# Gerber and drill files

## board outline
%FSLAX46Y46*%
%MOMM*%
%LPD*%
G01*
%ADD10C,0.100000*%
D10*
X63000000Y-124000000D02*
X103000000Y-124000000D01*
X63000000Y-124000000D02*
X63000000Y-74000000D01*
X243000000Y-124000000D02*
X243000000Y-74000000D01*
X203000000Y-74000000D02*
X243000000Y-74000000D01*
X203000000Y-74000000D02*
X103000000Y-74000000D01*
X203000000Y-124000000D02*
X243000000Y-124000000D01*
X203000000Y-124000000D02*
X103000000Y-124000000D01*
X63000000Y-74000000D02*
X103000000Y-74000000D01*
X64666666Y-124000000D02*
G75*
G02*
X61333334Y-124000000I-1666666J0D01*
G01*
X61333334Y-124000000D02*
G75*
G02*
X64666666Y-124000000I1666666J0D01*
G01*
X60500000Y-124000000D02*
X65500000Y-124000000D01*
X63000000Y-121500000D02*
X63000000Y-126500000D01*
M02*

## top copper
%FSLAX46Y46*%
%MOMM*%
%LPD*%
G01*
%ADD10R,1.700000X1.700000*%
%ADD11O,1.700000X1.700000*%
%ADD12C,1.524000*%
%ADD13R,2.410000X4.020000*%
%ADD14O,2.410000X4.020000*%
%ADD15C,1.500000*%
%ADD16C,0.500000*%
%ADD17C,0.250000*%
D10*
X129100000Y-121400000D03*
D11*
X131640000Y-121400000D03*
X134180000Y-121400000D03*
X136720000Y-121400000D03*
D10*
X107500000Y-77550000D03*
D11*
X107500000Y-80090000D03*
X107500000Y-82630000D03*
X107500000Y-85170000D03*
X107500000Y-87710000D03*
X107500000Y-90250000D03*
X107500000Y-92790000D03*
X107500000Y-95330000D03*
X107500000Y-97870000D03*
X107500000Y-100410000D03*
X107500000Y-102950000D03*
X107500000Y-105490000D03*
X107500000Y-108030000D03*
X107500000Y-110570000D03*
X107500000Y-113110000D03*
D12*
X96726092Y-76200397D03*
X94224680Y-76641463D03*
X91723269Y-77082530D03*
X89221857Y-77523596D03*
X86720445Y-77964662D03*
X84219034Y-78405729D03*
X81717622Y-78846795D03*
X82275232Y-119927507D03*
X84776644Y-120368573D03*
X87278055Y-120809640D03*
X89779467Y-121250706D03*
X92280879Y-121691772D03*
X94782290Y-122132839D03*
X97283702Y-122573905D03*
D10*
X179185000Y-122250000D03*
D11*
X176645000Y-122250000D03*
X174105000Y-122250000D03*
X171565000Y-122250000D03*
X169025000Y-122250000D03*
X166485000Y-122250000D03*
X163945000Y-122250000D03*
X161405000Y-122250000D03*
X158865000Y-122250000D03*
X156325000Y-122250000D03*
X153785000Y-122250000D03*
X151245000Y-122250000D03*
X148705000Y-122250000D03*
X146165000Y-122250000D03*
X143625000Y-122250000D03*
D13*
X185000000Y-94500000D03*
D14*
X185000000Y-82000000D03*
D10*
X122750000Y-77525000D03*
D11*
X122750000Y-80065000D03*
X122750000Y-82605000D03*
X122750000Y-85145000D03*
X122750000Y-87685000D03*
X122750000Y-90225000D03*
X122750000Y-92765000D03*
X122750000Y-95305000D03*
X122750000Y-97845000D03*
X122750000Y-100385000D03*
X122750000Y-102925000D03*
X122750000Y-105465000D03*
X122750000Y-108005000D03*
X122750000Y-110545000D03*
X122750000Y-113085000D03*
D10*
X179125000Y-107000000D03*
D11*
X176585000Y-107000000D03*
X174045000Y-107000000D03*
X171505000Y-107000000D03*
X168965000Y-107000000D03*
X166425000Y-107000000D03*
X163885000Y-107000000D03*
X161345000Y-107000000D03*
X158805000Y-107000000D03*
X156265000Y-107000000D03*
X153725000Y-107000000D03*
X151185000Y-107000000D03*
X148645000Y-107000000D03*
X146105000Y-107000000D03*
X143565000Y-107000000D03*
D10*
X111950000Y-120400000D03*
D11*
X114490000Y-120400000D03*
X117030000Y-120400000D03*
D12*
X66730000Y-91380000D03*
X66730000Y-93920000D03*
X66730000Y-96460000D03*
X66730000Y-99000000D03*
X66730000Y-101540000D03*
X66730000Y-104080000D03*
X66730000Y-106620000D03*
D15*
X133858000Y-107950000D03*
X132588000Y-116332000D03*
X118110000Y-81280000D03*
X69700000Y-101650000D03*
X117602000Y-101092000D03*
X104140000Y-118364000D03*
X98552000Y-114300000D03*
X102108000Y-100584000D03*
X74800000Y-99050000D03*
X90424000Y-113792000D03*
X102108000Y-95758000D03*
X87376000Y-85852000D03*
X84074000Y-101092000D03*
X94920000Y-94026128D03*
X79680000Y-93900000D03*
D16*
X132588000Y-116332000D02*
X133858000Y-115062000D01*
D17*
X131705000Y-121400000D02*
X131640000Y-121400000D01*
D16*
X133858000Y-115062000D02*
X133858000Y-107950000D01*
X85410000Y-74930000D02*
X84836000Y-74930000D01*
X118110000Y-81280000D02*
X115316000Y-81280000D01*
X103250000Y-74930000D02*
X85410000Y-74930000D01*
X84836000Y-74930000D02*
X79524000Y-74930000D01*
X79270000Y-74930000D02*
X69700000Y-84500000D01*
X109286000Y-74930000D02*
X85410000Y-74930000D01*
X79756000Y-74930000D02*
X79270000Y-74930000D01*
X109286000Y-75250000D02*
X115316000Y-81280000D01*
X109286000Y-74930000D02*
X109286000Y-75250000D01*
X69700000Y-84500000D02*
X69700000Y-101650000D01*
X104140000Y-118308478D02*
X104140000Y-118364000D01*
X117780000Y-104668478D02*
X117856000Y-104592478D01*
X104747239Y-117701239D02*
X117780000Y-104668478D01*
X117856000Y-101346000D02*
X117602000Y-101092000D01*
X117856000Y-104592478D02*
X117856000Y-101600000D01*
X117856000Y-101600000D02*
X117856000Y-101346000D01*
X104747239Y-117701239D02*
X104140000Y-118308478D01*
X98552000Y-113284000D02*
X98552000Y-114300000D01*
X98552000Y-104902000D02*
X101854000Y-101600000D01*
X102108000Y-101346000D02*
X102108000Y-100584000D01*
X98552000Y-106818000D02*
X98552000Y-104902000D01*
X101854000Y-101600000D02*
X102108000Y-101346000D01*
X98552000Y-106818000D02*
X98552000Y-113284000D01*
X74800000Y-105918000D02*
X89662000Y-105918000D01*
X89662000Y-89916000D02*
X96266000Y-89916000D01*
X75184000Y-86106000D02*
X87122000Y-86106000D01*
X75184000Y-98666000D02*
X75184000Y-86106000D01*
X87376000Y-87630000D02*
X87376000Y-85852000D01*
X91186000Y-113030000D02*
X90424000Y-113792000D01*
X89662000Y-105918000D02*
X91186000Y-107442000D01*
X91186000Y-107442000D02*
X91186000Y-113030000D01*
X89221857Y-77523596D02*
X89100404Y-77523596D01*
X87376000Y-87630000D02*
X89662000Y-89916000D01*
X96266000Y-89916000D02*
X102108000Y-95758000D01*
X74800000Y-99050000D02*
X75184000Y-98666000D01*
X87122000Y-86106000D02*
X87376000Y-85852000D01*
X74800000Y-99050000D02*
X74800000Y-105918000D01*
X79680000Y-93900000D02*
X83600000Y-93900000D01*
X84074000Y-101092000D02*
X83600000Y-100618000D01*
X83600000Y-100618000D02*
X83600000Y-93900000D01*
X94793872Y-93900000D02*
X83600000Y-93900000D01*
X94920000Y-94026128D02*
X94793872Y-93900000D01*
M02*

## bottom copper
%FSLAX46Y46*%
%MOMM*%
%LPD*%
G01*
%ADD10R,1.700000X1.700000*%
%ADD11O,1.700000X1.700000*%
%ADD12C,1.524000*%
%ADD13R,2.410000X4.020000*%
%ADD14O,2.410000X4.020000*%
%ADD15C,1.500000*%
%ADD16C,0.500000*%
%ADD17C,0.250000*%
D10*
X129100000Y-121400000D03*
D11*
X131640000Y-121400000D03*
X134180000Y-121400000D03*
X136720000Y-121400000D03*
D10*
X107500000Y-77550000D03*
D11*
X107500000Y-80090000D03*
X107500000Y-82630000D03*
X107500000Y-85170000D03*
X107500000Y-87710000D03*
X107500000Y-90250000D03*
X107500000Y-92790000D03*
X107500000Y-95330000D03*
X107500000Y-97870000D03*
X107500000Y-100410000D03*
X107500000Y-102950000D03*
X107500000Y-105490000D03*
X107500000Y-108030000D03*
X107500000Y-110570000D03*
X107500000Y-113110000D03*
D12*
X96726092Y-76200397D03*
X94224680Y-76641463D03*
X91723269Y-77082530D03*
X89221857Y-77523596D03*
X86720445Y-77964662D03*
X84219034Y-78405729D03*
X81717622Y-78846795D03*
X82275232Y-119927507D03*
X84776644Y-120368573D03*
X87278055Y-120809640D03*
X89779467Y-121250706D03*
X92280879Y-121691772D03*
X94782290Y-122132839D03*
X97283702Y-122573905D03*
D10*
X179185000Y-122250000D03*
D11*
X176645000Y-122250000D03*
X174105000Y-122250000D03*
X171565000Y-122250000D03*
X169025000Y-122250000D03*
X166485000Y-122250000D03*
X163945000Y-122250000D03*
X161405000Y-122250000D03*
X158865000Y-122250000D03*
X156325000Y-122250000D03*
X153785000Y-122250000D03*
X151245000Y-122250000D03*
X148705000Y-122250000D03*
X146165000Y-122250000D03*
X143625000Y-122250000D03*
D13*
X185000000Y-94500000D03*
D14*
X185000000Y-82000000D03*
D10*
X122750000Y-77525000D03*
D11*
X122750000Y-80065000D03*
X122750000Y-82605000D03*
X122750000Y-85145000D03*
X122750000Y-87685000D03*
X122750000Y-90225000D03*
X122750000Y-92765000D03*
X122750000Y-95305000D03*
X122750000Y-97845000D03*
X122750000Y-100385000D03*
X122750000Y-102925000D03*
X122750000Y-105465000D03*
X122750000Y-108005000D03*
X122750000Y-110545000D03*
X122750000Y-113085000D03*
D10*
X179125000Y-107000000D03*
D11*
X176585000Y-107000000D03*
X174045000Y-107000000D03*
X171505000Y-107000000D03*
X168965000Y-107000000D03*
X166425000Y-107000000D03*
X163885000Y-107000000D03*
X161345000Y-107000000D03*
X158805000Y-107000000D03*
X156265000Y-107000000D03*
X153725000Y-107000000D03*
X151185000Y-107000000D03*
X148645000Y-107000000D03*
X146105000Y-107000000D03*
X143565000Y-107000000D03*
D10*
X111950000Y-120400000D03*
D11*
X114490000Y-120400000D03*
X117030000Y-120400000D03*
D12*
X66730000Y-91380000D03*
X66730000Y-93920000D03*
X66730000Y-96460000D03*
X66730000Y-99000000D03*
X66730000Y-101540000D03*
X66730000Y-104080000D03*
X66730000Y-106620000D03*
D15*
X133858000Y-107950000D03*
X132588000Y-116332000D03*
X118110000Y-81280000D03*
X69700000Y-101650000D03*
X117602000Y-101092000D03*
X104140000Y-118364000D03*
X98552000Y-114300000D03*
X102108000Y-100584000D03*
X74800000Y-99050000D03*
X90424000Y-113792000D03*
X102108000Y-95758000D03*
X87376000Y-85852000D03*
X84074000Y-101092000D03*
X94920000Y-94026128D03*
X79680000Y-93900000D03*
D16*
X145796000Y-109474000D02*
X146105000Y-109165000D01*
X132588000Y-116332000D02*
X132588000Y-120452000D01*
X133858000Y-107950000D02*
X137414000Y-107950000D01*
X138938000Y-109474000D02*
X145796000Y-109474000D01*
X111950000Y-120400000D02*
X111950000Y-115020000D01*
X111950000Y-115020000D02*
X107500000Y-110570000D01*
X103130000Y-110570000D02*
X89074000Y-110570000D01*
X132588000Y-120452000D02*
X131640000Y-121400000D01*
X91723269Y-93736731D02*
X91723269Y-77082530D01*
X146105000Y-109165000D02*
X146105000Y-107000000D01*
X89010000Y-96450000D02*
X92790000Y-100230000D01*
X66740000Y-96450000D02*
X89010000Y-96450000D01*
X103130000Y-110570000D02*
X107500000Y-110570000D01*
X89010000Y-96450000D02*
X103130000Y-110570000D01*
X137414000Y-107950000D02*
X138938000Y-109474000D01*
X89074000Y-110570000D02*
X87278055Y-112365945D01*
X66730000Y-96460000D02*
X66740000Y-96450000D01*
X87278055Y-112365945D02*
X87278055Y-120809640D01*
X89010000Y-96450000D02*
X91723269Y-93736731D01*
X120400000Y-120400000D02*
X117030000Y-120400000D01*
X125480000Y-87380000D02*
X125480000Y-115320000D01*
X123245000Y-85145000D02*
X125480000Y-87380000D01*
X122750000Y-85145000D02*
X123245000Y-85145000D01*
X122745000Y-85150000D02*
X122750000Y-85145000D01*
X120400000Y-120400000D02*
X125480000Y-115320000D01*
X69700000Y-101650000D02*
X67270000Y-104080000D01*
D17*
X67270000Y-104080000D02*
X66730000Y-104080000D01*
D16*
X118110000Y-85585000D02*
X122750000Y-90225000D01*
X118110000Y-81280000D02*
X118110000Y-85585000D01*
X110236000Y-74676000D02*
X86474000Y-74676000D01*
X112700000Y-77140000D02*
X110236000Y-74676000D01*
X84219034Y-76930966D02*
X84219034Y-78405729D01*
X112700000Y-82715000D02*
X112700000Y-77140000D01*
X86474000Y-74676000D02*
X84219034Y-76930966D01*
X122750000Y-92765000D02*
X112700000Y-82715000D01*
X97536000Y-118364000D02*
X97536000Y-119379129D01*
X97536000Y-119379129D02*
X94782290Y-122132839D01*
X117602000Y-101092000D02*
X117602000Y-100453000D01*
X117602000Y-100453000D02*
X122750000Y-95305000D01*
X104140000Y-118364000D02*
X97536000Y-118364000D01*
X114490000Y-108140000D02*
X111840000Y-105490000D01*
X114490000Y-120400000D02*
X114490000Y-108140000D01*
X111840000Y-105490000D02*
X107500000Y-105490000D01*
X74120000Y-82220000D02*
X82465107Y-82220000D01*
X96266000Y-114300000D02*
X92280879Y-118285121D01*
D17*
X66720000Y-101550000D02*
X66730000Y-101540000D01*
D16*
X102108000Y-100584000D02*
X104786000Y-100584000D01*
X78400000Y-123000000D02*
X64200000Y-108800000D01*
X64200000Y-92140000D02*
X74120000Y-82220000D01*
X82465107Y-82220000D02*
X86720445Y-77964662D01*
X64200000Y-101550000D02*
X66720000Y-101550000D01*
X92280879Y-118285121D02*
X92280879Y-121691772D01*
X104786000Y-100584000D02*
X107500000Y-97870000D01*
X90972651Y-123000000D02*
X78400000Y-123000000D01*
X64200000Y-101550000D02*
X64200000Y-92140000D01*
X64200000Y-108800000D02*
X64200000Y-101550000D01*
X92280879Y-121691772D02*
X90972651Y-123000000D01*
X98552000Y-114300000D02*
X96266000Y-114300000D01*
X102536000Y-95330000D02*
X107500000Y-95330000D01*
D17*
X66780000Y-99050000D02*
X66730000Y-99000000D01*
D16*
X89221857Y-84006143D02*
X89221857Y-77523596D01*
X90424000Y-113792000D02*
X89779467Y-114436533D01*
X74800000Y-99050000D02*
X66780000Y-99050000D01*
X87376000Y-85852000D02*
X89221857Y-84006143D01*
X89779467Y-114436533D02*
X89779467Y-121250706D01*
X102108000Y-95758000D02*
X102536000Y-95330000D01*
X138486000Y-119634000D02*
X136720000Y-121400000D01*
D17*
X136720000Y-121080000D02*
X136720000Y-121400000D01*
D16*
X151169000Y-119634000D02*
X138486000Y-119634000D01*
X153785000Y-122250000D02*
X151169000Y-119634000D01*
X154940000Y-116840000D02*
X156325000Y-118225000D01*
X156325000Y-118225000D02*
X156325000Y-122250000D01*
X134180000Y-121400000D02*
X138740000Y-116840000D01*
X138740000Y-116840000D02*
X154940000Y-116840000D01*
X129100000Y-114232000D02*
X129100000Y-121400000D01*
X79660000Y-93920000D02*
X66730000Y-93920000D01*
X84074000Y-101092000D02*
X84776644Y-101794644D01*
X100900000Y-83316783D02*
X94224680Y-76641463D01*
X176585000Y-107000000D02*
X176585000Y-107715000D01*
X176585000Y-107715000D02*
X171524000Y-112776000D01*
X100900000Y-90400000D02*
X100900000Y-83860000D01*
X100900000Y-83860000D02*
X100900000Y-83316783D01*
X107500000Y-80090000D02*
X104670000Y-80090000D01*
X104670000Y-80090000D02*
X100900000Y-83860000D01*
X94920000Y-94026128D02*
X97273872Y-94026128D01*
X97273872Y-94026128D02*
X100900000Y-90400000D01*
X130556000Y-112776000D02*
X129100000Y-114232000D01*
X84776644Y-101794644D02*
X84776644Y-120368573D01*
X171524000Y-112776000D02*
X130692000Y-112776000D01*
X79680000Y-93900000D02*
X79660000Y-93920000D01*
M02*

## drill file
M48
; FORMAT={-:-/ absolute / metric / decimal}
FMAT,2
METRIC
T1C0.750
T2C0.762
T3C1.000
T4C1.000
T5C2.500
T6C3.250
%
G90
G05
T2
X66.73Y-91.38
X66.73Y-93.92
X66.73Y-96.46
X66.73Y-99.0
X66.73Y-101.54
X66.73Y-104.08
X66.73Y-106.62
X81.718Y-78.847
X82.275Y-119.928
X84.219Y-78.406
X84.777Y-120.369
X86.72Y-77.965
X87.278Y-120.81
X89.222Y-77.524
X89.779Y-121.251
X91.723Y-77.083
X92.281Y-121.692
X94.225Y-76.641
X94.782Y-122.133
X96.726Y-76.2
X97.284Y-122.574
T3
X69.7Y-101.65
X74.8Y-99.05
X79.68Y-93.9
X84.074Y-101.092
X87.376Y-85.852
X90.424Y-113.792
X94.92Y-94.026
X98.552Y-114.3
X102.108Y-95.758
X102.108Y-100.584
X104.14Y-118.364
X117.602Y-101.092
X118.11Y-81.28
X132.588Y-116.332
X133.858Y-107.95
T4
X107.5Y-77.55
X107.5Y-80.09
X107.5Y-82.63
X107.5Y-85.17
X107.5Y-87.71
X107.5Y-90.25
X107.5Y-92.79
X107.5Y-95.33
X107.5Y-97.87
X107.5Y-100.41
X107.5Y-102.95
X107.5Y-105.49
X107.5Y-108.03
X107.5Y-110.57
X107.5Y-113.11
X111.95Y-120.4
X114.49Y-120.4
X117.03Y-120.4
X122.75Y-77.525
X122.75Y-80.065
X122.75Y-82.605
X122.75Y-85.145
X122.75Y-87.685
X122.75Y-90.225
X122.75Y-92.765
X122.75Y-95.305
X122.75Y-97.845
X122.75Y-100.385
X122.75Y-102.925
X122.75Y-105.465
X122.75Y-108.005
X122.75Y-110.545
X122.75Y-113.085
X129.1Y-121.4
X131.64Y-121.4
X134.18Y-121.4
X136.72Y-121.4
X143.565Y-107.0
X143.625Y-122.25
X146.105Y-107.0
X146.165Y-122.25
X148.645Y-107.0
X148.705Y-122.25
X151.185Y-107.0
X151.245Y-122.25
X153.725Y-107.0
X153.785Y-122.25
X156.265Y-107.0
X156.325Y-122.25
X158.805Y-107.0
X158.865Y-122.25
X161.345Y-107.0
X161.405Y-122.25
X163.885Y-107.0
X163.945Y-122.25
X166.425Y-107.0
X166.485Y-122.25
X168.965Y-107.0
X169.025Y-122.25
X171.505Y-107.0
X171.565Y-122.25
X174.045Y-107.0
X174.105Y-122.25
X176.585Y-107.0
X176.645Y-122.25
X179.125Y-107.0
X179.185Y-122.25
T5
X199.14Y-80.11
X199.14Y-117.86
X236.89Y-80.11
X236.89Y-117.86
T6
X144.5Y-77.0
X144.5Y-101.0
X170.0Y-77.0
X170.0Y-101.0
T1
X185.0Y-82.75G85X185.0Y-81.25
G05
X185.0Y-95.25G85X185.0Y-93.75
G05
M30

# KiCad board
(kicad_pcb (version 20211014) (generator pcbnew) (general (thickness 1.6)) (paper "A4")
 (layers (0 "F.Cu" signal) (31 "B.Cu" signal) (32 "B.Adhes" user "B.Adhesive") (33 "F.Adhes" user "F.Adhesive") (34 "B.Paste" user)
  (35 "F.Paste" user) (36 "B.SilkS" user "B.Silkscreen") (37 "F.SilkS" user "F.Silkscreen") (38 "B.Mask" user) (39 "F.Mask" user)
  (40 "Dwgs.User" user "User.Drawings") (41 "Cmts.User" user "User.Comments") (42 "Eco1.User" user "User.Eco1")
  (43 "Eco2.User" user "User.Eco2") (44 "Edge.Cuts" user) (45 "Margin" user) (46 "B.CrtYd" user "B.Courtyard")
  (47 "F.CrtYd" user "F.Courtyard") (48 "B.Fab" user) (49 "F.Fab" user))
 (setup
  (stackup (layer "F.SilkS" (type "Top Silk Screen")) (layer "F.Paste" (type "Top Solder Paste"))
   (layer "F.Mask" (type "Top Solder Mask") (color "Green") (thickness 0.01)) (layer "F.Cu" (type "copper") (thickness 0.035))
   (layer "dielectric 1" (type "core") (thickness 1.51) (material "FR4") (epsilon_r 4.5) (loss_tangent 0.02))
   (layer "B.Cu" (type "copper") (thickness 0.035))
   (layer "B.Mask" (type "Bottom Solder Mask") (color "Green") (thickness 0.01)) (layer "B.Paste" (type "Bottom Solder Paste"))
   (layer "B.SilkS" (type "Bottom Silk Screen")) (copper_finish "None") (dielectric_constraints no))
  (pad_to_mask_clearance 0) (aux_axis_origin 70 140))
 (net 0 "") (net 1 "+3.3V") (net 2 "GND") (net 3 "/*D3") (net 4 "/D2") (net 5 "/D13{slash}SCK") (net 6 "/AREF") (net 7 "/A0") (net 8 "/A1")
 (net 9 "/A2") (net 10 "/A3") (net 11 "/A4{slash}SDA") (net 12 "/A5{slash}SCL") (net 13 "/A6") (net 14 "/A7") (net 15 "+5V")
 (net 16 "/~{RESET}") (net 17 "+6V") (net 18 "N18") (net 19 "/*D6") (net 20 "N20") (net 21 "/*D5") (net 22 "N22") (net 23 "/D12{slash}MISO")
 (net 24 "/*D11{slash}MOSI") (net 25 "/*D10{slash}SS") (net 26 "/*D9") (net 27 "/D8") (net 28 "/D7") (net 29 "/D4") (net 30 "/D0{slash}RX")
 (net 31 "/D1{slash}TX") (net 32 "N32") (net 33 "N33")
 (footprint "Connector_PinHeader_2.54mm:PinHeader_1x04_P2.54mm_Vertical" (layer "F.Cu") (at 129.1 121.4 90)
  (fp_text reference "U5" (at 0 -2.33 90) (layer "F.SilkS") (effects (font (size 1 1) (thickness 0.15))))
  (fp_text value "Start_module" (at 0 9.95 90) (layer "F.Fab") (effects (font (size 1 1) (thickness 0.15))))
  (pad "1" thru_hole rect (at 0 0 90) (size 1.7 1.7) (drill 1) (layers *.Cu *.Mask) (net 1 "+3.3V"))
  (pad "2" thru_hole oval (at 0 2.54 90) (size 1.7 1.7) (drill 1) (layers *.Cu *.Mask) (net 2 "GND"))
  (pad "3" thru_hole oval (at 0 5.08 90) (size 1.7 1.7) (drill 1) (layers *.Cu *.Mask) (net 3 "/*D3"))
  (pad "4" thru_hole oval (at 0 7.62 90) (size 1.7 1.7) (drill 1) (layers *.Cu *.Mask) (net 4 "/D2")))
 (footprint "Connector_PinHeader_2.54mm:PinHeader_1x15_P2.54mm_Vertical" (layer "F.Cu") (at 107.5 77.55)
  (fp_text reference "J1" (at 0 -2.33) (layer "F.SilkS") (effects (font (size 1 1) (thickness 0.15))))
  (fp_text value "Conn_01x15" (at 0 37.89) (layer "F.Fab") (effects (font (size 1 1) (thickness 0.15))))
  (pad "1" thru_hole rect (at 0 0) (size 1.7 1.7) (drill 1) (layers *.Cu *.Mask) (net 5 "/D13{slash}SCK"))
  (pad "2" thru_hole oval (at 0 2.54) (size 1.7 1.7) (drill 1) (layers *.Cu *.Mask) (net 1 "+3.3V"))
  (pad "3" thru_hole oval (at 0 5.08) (size 1.7 1.7) (drill 1) (layers *.Cu *.Mask) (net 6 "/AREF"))
  (pad "4" thru_hole oval (at 0 7.62) (size 1.7 1.7) (drill 1) (layers *.Cu *.Mask) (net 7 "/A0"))
  (pad "5" thru_hole oval (at 0 10.16) (size 1.7 1.7) (drill 1) (layers *.Cu *.Mask) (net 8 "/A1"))
  (pad "6" thru_hole oval (at 0 12.7) (size 1.7 1.7) (drill 1) (layers *.Cu *.Mask) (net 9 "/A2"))
  (pad "7" thru_hole oval (at 0 15.24) (size 1.7 1.7) (drill 1) (layers *.Cu *.Mask) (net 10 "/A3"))
  (pad "8" thru_hole oval (at 0 17.78) (size 1.7 1.7) (drill 1) (layers *.Cu *.Mask) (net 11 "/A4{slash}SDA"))
  (pad "9" thru_hole oval (at 0 20.32) (size 1.7 1.7) (drill 1) (layers *.Cu *.Mask) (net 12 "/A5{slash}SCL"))
  (pad "10" thru_hole oval (at 0 22.86) (size 1.7 1.7) (drill 1) (layers *.Cu *.Mask) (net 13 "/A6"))
  (pad "11" thru_hole oval (at 0 25.4) (size 1.7 1.7) (drill 1) (layers *.Cu *.Mask) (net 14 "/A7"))
  (pad "12" thru_hole oval (at 0 27.94) (size 1.7 1.7) (drill 1) (layers *.Cu *.Mask) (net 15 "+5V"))
  (pad "13" thru_hole oval (at 0 30.48) (size 1.7 1.7) (drill 1) (layers *.Cu *.Mask) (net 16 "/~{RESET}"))
  (pad "14" thru_hole oval (at 0 33.02) (size 1.7 1.7) (drill 1) (layers *.Cu *.Mask) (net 2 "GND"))
  (pad "15" thru_hole oval (at 0 35.56) (size 1.7 1.7) (drill 1) (layers *.Cu *.Mask) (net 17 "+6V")))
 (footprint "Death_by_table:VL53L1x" (layer "F.Cu") (at 96.726092 76.200397 -170)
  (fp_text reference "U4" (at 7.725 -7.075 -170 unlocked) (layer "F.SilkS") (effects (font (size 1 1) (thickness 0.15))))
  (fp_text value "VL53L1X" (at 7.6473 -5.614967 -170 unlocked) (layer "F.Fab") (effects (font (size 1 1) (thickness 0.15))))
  (pad "1" thru_hole circle (at 0 0 190) (size 1.524 1.524) (drill 0.762) (layers *.Cu *.Mask) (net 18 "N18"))
  (pad "2" thru_hole circle (at 2.54 0 190) (size 1.524 1.524) (drill 0.762) (layers *.Cu *.Mask) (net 1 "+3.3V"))
  (pad "3" thru_hole circle (at 5.08 0 190) (size 1.524 1.524) (drill 0.762) (layers *.Cu *.Mask) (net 2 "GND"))
  (pad "4" thru_hole circle (at 7.62 0 190) (size 1.524 1.524) (drill 0.762) (layers *.Cu *.Mask) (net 11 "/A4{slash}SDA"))
  (pad "5" thru_hole circle (at 10.16 0 190) (size 1.524 1.524) (drill 0.762) (layers *.Cu *.Mask) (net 12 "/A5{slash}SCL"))
  (pad "6" thru_hole circle (at 12.7 0 190) (size 1.524 1.524) (drill 0.762) (layers *.Cu *.Mask) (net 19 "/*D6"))
  (pad "7" thru_hole circle (at 15.24 0 190) (size 1.524 1.524) (drill 0.762) (layers *.Cu *.Mask) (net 18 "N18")))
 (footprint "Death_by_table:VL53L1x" (layer "F.Cu") (at 82.275232 119.927507 -10)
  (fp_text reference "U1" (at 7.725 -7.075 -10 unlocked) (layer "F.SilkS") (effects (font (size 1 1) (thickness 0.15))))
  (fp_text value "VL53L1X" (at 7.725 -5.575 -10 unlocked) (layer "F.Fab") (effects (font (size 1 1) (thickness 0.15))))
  (pad "1" thru_hole circle (at 0 0 350) (size 1.524 1.524) (drill 0.762) (layers *.Cu *.Mask) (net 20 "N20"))
  (pad "2" thru_hole circle (at 2.54 0 350) (size 1.524 1.524) (drill 0.762) (layers *.Cu *.Mask) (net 1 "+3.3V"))
  (pad "3" thru_hole circle (at 5.08 0 350) (size 1.524 1.524) (drill 0.762) (layers *.Cu *.Mask) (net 2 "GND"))
  (pad "4" thru_hole circle (at 7.62 0 350) (size 1.524 1.524) (drill 0.762) (layers *.Cu *.Mask) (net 11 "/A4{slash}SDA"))
  (pad "5" thru_hole circle (at 10.16 0 350) (size 1.524 1.524) (drill 0.762) (layers *.Cu *.Mask) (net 12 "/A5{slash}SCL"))
  (pad "6" thru_hole circle (at 12.7 0 350) (size 1.524 1.524) (drill 0.762) (layers *.Cu *.Mask) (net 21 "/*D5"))
  (pad "7" thru_hole circle (at 15.24 0 350) (size 1.524 1.524) (drill 0.762) (layers *.Cu *.Mask) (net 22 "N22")))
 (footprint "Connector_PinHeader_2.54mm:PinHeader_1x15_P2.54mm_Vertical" (layer "F.Cu") (at 179.185 122.25 -90)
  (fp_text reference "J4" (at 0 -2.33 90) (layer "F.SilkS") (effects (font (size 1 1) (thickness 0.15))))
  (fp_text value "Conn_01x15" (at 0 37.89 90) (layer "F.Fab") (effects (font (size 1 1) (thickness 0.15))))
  (pad "1" thru_hole rect (at 0 0 270) (size 1.7 1.7) (drill 1) (layers *.Cu *.Mask) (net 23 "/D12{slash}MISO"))
  (pad "2" thru_hole oval (at 0 2.54 270) (size 1.7 1.7) (drill 1) (layers *.Cu *.Mask) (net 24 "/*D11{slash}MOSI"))
  (pad "3" thru_hole oval (at 0 5.08 270) (size 1.7 1.7) (drill 1) (layers *.Cu *.Mask) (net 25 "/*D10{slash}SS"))
  (pad "4" thru_hole oval (at 0 7.62 270) (size 1.7 1.7) (drill 1) (layers *.Cu *.Mask) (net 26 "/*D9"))
  (pad "5" thru_hole oval (at 0 10.16 270) (size 1.7 1.7) (drill 1) (layers *.Cu *.Mask) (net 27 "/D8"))
  (pad "6" thru_hole oval (at 0 12.7 270) (size 1.7 1.7) (drill 1) (layers *.Cu *.Mask) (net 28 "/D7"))
  (pad "7" thru_hole oval (at 0 15.24 270) (size 1.7 1.7) (drill 1) (layers *.Cu *.Mask) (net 19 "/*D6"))
  (pad "8" thru_hole oval (at 0 17.78 270) (size 1.7 1.7) (drill 1) (layers *.Cu *.Mask) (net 21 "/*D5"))
  (pad "9" thru_hole oval (at 0 20.32 270) (size 1.7 1.7) (drill 1) (layers *.Cu *.Mask) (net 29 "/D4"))
  (pad "10" thru_hole oval (at 0 22.86 270) (size 1.7 1.7) (drill 1) (layers *.Cu *.Mask) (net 3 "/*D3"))
  (pad "11" thru_hole oval (at 0 25.4 270) (size 1.7 1.7) (drill 1) (layers *.Cu *.Mask) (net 4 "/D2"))
  (pad "12" thru_hole oval (at 0 27.94 270) (size 1.7 1.7) (drill 1) (layers *.Cu *.Mask) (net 2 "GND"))
  (pad "13" thru_hole oval (at 0 30.48 270) (size 1.7 1.7) (drill 1) (layers *.Cu *.Mask) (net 16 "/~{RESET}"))
  (pad "14" thru_hole oval (at 0 33.02 270) (size 1.7 1.7) (drill 1) (layers *.Cu *.Mask) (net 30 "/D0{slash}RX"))
  (pad "15" thru_hole oval (at 0 35.56 270) (size 1.7 1.7) (drill 1) (layers *.Cu *.Mask) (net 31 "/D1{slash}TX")))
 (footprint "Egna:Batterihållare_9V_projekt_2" (layer "F.Cu") (at 185 74 180)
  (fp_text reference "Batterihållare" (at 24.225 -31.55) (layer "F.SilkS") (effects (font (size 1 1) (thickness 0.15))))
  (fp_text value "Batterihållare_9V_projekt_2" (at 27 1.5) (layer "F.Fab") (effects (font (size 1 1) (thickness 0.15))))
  (pad "" np_thru_hole circle (at 15 -27 180) (size 2.3 2.3) (drill 3.25) (layers F&B.Cu *.Mask))
  (pad "" np_thru_hole circle (at 40.5 -3 180) (size 2.3 2.3) (drill 3.25) (layers F&B.Cu *.Mask))
  (pad "" np_thru_hole circle (at 15 -3 180) (size 2.3 2.3) (drill 3.25) (layers F&B.Cu *.Mask))
  (pad "" np_thru_hole circle (at 40.5 -27 180) (size 2.3 2.3) (drill 3.25) (layers F&B.Cu *.Mask))
  (pad "1" thru_hole rect (at 0 -20.5 180) (size 2.41 4.02) (drill oval 0.75 2.25) (layers *.Cu *.Mask))
  (pad "2" thru_hole oval (at 0 -8 180) (size 2.41 4.02) (drill oval 0.75 2.25) (layers *.Cu *.Mask)))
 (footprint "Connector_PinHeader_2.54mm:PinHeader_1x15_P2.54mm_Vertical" (layer "F.Cu") (at 122.75 77.525)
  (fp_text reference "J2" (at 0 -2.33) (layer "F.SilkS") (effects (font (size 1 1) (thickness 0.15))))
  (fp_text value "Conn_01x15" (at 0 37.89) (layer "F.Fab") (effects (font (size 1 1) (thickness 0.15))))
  (pad "1" thru_hole rect (at 0 0) (size 1.7 1.7) (drill 1) (layers *.Cu *.Mask) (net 23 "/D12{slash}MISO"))
  (pad "2" thru_hole oval (at 0 2.54) (size 1.7 1.7) (drill 1) (layers *.Cu *.Mask) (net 24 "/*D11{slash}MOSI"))
  (pad "3" thru_hole oval (at 0 5.08) (size 1.7 1.7) (drill 1) (layers *.Cu *.Mask) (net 25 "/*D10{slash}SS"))
  (pad "4" thru_hole oval (at 0 7.62) (size 1.7 1.7) (drill 1) (layers *.Cu *.Mask) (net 26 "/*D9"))
  (pad "5" thru_hole oval (at 0 10.16) (size 1.7 1.7) (drill 1) (layers *.Cu *.Mask) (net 27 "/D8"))
  (pad "6" thru_hole oval (at 0 12.7) (size 1.7 1.7) (drill 1) (layers *.Cu *.Mask) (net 28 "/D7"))
  (pad "7" thru_hole oval (at 0 15.24) (size 1.7 1.7) (drill 1) (layers *.Cu *.Mask) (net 19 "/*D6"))
  (pad "8" thru_hole oval (at 0 17.78) (size 1.7 1.7) (drill 1) (layers *.Cu *.Mask) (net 21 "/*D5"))
  (pad "9" thru_hole oval (at 0 20.32) (size 1.7 1.7) (drill 1) (layers *.Cu *.Mask) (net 29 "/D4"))
  (pad "10" thru_hole oval (at 0 22.86) (size 1.7 1.7) (drill 1) (layers *.Cu *.Mask) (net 3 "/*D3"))
  (pad "11" thru_hole oval (at 0 25.4) (size 1.7 1.7) (drill 1) (layers *.Cu *.Mask) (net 4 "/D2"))
  (pad "12" thru_hole oval (at 0 27.94) (size 1.7 1.7) (drill 1) (layers *.Cu *.Mask) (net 2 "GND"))
  (pad "13" thru_hole oval (at 0 30.48) (size 1.7 1.7) (drill 1) (layers *.Cu *.Mask) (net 16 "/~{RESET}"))
  (pad "14" thru_hole oval (at 0 33.02) (size 1.7 1.7) (drill 1) (layers *.Cu *.Mask) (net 30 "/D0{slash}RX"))
  (pad "15" thru_hole oval (at 0 35.56) (size 1.7 1.7) (drill 1) (layers *.Cu *.Mask) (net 31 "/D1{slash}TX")))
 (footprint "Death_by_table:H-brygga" (layer "F.Cu") (at 195.14 121.86)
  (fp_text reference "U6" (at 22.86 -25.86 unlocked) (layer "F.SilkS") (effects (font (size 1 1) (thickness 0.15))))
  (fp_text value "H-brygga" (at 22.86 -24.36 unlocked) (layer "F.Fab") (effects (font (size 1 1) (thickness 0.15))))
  (pad "" np_thru_hole circle (at 4 -4) (size 2.5 2.5) (drill 2.5) (layers F&B.Cu *.Mask))
  (pad "" np_thru_hole circle (at 41.75 -41.75) (size 2.5 2.5) (drill 2.5) (layers F&B.Cu *.Mask))
  (pad "" np_thru_hole circle (at 4 -41.75) (size 2.5 2.5) (drill 2.5) (layers F&B.Cu *.Mask))
  (pad "" np_thru_hole circle (at 41.75 -4) (size 2.5 2.5) (drill 2.5) (layers F&B.Cu *.Mask)))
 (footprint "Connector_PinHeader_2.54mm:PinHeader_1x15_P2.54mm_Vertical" (layer "F.Cu") (at 179.125 107 -90)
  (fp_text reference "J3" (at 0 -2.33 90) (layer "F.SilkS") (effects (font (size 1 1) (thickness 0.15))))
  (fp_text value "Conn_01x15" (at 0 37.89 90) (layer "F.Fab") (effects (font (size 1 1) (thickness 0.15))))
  (pad "1" thru_hole rect (at 0 0 270) (size 1.7 1.7) (drill 1) (layers *.Cu *.Mask) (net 5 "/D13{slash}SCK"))
  (pad "2" thru_hole oval (at 0 2.54 270) (size 1.7 1.7) (drill 1) (layers *.Cu *.Mask) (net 1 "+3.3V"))
  (pad "3" thru_hole oval (at 0 5.08 270) (size 1.7 1.7) (drill 1) (layers *.Cu *.Mask) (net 6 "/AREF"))
  (pad "4" thru_hole oval (at 0 7.62 270) (size 1.7 1.7) (drill 1) (layers *.Cu *.Mask) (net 7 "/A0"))
  (pad "5" thru_hole oval (at 0 10.16 270) (size 1.7 1.7) (drill 1) (layers *.Cu *.Mask) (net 8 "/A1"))
  (pad "6" thru_hole oval (at 0 12.7 270) (size 1.7 1.7) (drill 1) (layers *.Cu *.Mask) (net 9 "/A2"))
  (pad "7" thru_hole oval (at 0 15.24 270) (size 1.7 1.7) (drill 1) (layers *.Cu *.Mask) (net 10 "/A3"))
  (pad "8" thru_hole oval (at 0 17.78 270) (size 1.7 1.7) (drill 1) (layers *.Cu *.Mask) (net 11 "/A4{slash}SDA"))
  (pad "9" thru_hole oval (at 0 20.32 270) (size 1.7 1.7) (drill 1) (layers *.Cu *.Mask) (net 12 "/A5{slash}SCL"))
  (pad "10" thru_hole oval (at 0 22.86 270) (size 1.7 1.7) (drill 1) (layers *.Cu *.Mask) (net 13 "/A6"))
  (pad "11" thru_hole oval (at 0 25.4 270) (size 1.7 1.7) (drill 1) (layers *.Cu *.Mask) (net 14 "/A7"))
  (pad "12" thru_hole oval (at 0 27.94 270) (size 1.7 1.7) (drill 1) (layers *.Cu *.Mask) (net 15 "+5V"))
  (pad "13" thru_hole oval (at 0 30.48 270) (size 1.7 1.7) (drill 1) (layers *.Cu *.Mask) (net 16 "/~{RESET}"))
  (pad "14" thru_hole oval (at 0 33.02 270) (size 1.7 1.7) (drill 1) (layers *.Cu *.Mask) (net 2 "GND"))
  (pad "15" thru_hole oval (at 0 35.56 270) (size 1.7 1.7) (drill 1) (layers *.Cu *.Mask) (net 17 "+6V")))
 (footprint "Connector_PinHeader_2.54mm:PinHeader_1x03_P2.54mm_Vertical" (layer "F.Cu") (at 111.95 120.4 90)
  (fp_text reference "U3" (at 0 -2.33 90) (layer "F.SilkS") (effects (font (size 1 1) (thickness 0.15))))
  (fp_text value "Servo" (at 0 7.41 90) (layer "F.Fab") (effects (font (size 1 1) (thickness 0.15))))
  (pad "1" thru_hole rect (at 0 0 90) (size 1.7 1.7) (drill 1) (layers *.Cu *.Mask) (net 2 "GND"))
  (pad "2" thru_hole oval (at 0 2.54 90) (size 1.7 1.7) (drill 1) (layers *.Cu *.Mask) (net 15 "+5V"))
  (pad "3" thru_hole oval (at 0 5.08 90) (size 1.7 1.7) (drill 1) (layers *.Cu *.Mask) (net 26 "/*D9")))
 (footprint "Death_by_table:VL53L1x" (layer "F.Cu") (at 66.73 91.38 -90)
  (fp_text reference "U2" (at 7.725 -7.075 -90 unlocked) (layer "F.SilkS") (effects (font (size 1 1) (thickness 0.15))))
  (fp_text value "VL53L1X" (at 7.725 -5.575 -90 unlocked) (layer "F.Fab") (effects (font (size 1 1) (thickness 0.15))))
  (pad "1" thru_hole circle (at 0 0 270) (size 1.524 1.524) (drill 0.762) (layers *.Cu *.Mask) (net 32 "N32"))
  (pad "2" thru_hole circle (at 2.54 0 270) (size 1.524 1.524) (drill 0.762) (layers *.Cu *.Mask) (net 1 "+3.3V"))
  (pad "3" thru_hole circle (at 5.08 0 270) (size 1.524 1.524) (drill 0.762) (layers *.Cu *.Mask) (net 2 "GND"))
  (pad "4" thru_hole circle (at 7.62 0 270) (size 1.524 1.524) (drill 0.762) (layers *.Cu *.Mask) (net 11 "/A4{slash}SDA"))
  (pad "5" thru_hole circle (at 10.16 0 270) (size 1.524 1.524) (drill 0.762) (layers *.Cu *.Mask) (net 12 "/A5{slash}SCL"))
  (pad "6" thru_hole circle (at 12.7 0 270) (size 1.524 1.524) (drill 0.762) (layers *.Cu *.Mask) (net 28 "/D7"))
  (pad "7" thru_hole circle (at 15.24 0 270) (size 1.524 1.524) (drill 0.762) (layers *.Cu *.Mask) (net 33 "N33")))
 (gr_line (start 63 124) (end 103 124) (layer "Edge.Cuts") (width 0.1))
 (gr_line (start 63 124) (end 63 74) (layer "Edge.Cuts") (width 0.1))
 (gr_line (start 243 124) (end 243 74) (layer "Edge.Cuts") (width 0.1))
 (gr_line (start 203 74) (end 243 74) (layer "Edge.Cuts") (width 0.1))
 (gr_line (start 203 74) (end 103 74) (layer "Edge.Cuts") (width 0.1))
 (gr_line (start 203 124) (end 243 124) (layer "Edge.Cuts") (width 0.1))
 (gr_line (start 203 124) (end 103 124) (layer "Edge.Cuts") (width 0.1))
 (gr_line (start 63 74) (end 103 74) (layer "Edge.Cuts") (width 0.1))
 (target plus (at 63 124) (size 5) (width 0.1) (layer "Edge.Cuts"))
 (segment (start 132.588 116.332) (end 133.858 115.062) (width 0.5) (layer "F.Cu") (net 2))
 (segment (start 131.705 121.4) (end 131.64 121.4) (width 0.25) (layer "F.Cu") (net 2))
 (segment (start 133.858 115.062) (end 133.858 107.95) (width 0.5) (layer "F.Cu") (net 2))
 (via (at 133.858 107.95) (size 1.5) (drill 1) (layers "F.Cu" "B.Cu") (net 2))
 (via (at 132.588 116.332) (size 1.5) (drill 1) (layers "F.Cu" "B.Cu") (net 2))
 (segment (start 145.796 109.474) (end 146.105 109.165) (width 0.5) (layer "B.Cu") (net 2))
 (segment (start 132.588 116.332) (end 132.588 120.452) (width 0.5) (layer "B.Cu") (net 2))
 (segment (start 133.858 107.95) (end 137.414 107.95) (width 0.5) (layer "B.Cu") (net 2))
 (segment (start 138.938 109.474) (end 145.796 109.474) (width 0.5) (layer "B.Cu") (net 2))
 (segment (start 111.95 120.4) (end 111.95 115.02) (width 0.5) (layer "B.Cu") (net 2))
 (segment (start 111.95 115.02) (end 107.5 110.57) (width 0.5) (layer "B.Cu") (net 2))
 (segment (start 103.13 110.57) (end 89.074 110.57) (width 0.5) (layer "B.Cu") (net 2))
 (segment (start 132.588 120.452) (end 131.64 121.4) (width 0.5) (layer "B.Cu") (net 2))
 (segment (start 91.723269 93.736731) (end 91.723269 77.08253) (width 0.5) (layer "B.Cu") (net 2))
 (segment (start 146.105 109.165) (end 146.105 107) (width 0.5) (layer "B.Cu") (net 2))
 (segment (start 89.01 96.45) (end 92.79 100.23) (width 0.5) (layer "B.Cu") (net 2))
 (segment (start 66.74 96.45) (end 89.01 96.45) (width 0.5) (layer "B.Cu") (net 2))
 (segment (start 103.13 110.57) (end 107.5 110.57) (width 0.5) (layer "B.Cu") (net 2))
 (segment (start 89.01 96.45) (end 103.13 110.57) (width 0.5) (layer "B.Cu") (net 2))
 (segment (start 137.414 107.95) (end 138.938 109.474) (width 0.5) (layer "B.Cu") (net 2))
 (segment (start 89.074 110.57) (end 87.278055 112.365945) (width 0.5) (layer "B.Cu") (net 2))
 (segment (start 66.73 96.46) (end 66.74 96.45) (width 0.5) (layer "B.Cu") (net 2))
 (segment (start 87.278055 112.365945) (end 87.278055 120.80964) (width 0.5) (layer "B.Cu") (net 2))
 (segment (start 89.01 96.45) (end 91.723269 93.736731) (width 0.5) (layer "B.Cu") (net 2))
 (segment (start 120.4 120.4) (end 117.03 120.4) (width 0.5) (layer "B.Cu") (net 26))
 (segment (start 125.48 87.38) (end 125.48 115.32) (width 0.5) (layer "B.Cu") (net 26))
 (segment (start 123.245 85.145) (end 125.48 87.38) (width 0.5) (layer "B.Cu") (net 26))
 (segment (start 122.75 85.145) (end 123.245 85.145) (width 0.5) (layer "B.Cu") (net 26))
 (segment (start 122.745 85.15) (end 122.75 85.145) (width 0.5) (layer "B.Cu") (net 26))
 (segment (start 120.4 120.4) (end 125.48 115.32) (width 0.5) (layer "B.Cu") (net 26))
 (segment (start 85.41 74.93) (end 84.836 74.93) (width 0.5) (layer "F.Cu") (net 28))
 (segment (start 118.11 81.28) (end 115.316 81.28) (width 0.5) (layer "F.Cu") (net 28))
 (segment (start 103.25 74.93) (end 85.41 74.93) (width 0.5) (layer "F.Cu") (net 28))
 (segment (start 84.836 74.93) (end 79.524 74.93) (width 0.5) (layer "F.Cu") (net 28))
 (segment (start 79.27 74.93) (end 69.7 84.5) (width 0.5) (layer "F.Cu") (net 28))
 (segment (start 109.286 74.93) (end 85.41 74.93) (width 0.5) (layer "F.Cu") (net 28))
 (segment (start 79.756 74.93) (end 79.27 74.93) (width 0.5) (layer "F.Cu") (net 28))
 (segment (start 109.286 75.25) (end 115.316 81.28) (width 0.5) (layer "F.Cu") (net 28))
 (segment (start 109.286 74.93) (end 109.286 75.25) (width 0.5) (layer "F.Cu") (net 28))
 (segment (start 69.7 84.5) (end 69.7 101.65) (width 0.5) (layer "F.Cu") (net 28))
 (via (at 118.11 81.28) (size 1.5) (drill 1) (layers "F.Cu" "B.Cu") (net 28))
 (via (at 69.7 101.65) (size 1.5) (drill 1) (layers "F.Cu" "B.Cu") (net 28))
 (segment (start 69.7 101.65) (end 67.27 104.08) (width 0.5) (layer "B.Cu") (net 28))
 (segment (start 67.27 104.08) (end 66.73 104.08) (width 0.25) (layer "B.Cu") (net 28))
 (segment (start 118.11 85.585) (end 122.75 90.225) (width 0.5) (layer "B.Cu") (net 28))
 (segment (start 118.11 81.28) (end 118.11 85.585) (width 0.5) (layer "B.Cu") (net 28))
 (segment (start 110.236 74.676) (end 86.474 74.676) (width 0.5) (layer "B.Cu") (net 19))
 (segment (start 112.7 77.14) (end 110.236 74.676) (width 0.5) (layer "B.Cu") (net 19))
 (segment (start 84.219034 76.930966) (end 84.219034 78.405729) (width 0.5) (layer "B.Cu") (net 19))
 (segment (start 112.7 82.715) (end 112.7 77.14) (width 0.5) (layer "B.Cu") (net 19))
 (segment (start 86.474 74.676) (end 84.219034 76.930966) (width 0.5) (layer "B.Cu") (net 19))
 (segment (start 122.75 92.765) (end 112.7 82.715) (width 0.5) (layer "B.Cu") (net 19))
 (segment (start 104.14 118.308478) (end 104.14 118.364) (width 0.5) (layer "F.Cu") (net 21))
 (segment (start 117.78 104.668478) (end 117.856 104.592478) (width 0.5) (layer "F.Cu") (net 21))
 (segment (start 104.747239 117.701239) (end 117.78 104.668478) (width 0.5) (layer "F.Cu") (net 21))
 (segment (start 117.856 101.346) (end 117.602 101.092) (width 0.5) (layer "F.Cu") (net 21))
 (segment (start 117.856 104.592478) (end 117.856 101.6) (width 0.5) (layer "F.Cu") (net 21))
 (segment (start 117.856 101.6) (end 117.856 101.346) (width 0.5) (layer "F.Cu") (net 21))
 (segment (start 104.747239 117.701239) (end 104.14 118.308478) (width 0.5) (layer "F.Cu") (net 21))
 (via (at 117.602 101.092) (size 1.5) (drill 1) (layers "F.Cu" "B.Cu") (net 21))
 (via (at 104.14 118.364) (size 1.5) (drill 1) (layers "F.Cu" "B.Cu") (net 21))
 (segment (start 97.536 118.364) (end 97.536 119.379129) (width 0.5) (layer "B.Cu") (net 21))
 (segment (start 97.536 119.379129) (end 94.78229 122.132839) (width 0.5) (layer "B.Cu") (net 21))
 (segment (start 117.602 101.092) (end 117.602 100.453) (width 0.5) (layer "B.Cu") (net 21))
 (segment (start 117.602 100.453) (end 122.75 95.305) (width 0.5) (layer "B.Cu") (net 21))
 (segment (start 104.14 118.364) (end 97.536 118.364) (width 0.5) (layer "B.Cu") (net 21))
 (segment (start 114.49 108.14) (end 111.84 105.49) (width 0.5) (layer "B.Cu") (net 15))
 (segment (start 114.49 120.4) (end 114.49 108.14) (width 0.5) (layer "B.Cu") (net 15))
 (segment (start 111.84 105.49) (end 107.5 105.49) (width 0.5) (layer "B.Cu") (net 15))
 (segment (start 98.552 113.284) (end 98.552 114.3) (width 0.5) (layer "F.Cu") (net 12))
 (segment (start 98.552 104.902) (end 101.854 101.6) (width 0.5) (layer "F.Cu") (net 12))
 (segment (start 102.108 101.346) (end 102.108 100.584) (width 0.5) (layer "F.Cu") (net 12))
 (segment (start 98.552 106.818) (end 98.552 104.902) (width 0.5) (layer "F.Cu") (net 12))
 (segment (start 101.854 101.6) (end 102.108 101.346) (width 0.5) (layer "F.Cu") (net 12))
 (segment (start 98.552 106.818) (end 98.552 113.284) (width 0.5) (layer "F.Cu") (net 12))
 (via (at 98.552 114.3) (size 1.5) (drill 1) (layers "F.Cu" "B.Cu") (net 12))
 (via (at 102.108 100.584) (size 1.5) (drill 1) (layers "F.Cu" "B.Cu") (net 12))
 (segment (start 74.12 82.22) (end 82.465107 82.22) (width 0.5) (layer "B.Cu") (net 12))
 (segment (start 96.266 114.3) (end 92.280879 118.285121) (width 0.5) (layer "B.Cu") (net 12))
 (segment (start 66.72 101.55) (end 66.73 101.54) (width 0.25) (layer "B.Cu") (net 12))
 (segment (start 102.108 100.584) (end 104.786 100.584) (width 0.5) (layer "B.Cu") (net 12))
 (segment (start 78.4 123) (end 64.2 108.8) (width 0.5) (layer "B.Cu") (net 12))
 (segment (start 64.2 92.14) (end 74.12 82.22) (width 0.5) (layer "B.Cu") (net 12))
 (segment (start 82.465107 82.22) (end 86.720445 77.964662) (width 0.5) (layer "B.Cu") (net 12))
 (segment (start 64.2 101.55) (end 66.72 101.55) (width 0.5) (layer "B.Cu") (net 12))
 (segment (start 92.280879 118.285121) (end 92.280879 121.691772) (width 0.5) (layer "B.Cu") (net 12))
 (segment (start 104.786 100.584) (end 107.5 97.87) (width 0.5) (layer "B.Cu") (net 12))
 (segment (start 90.972651 123) (end 78.4 123) (width 0.5) (layer "B.Cu") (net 12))
 (segment (start 64.2 101.55) (end 64.2 92.14) (width 0.5) (layer "B.Cu") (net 12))
 (segment (start 64.2 108.8) (end 64.2 101.55) (width 0.5) (layer "B.Cu") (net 12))
 (segment (start 92.280879 121.691772) (end 90.972651 123) (width 0.5) (layer "B.Cu") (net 12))
 (segment (start 98.552 114.3) (end 96.266 114.3) (width 0.5) (layer "B.Cu") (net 12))
 (segment (start 74.8 105.918) (end 89.662 105.918) (width 0.5) (layer "F.Cu") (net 11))
 (segment (start 89.662 89.916) (end 96.266 89.916) (width 0.5) (layer "F.Cu") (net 11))
 (segment (start 75.184 86.106) (end 87.122 86.106) (width 0.5) (layer "F.Cu") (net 11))
 (segment (start 75.184 98.666) (end 75.184 86.106) (width 0.5) (layer "F.Cu") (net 11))
 (segment (start 87.376 87.63) (end 87.376 85.852) (width 0.5) (layer "F.Cu") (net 11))
 (segment (start 91.186 113.03) (end 90.424 113.792) (width 0.5) (layer "F.Cu") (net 11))
 (segment (start 89.662 105.918) (end 91.186 107.442) (width 0.5) (layer "F.Cu") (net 11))
 (segment (start 91.186 107.442) (end 91.186 113.03) (width 0.5) (layer "F.Cu") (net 11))
 (segment (start 89.221857 77.523596) (end 89.100404 77.523596) (width 0.5) (layer "F.Cu") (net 11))
 (segment (start 87.376 87.63) (end 89.662 89.916) (width 0.5) (layer "F.Cu") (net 11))
 (segment (start 96.266 89.916) (end 102.108 95.758) (width 0.5) (layer "F.Cu") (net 11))
 (segment (start 74.8 99.05) (end 75.184 98.666) (width 0.5) (layer "F.Cu") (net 11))
 (segment (start 87.122 86.106) (end 87.376 85.852) (width 0.5) (layer "F.Cu") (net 11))
 (segment (start 74.8 99.05) (end 74.8 105.918) (width 0.5) (layer "F.Cu") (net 11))
 (via (at 74.8 99.05) (size 1.5) (drill 1) (layers "F.Cu" "B.Cu") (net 11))
 (via (at 90.424 113.792) (size 1.5) (drill 1) (layers "F.Cu" "B.Cu") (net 11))
 (via (at 102.108 95.758) (size 1.5) (drill 1) (layers "F.Cu" "B.Cu") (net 11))
 (via (at 87.376 85.852) (size 1.5) (drill 1) (layers "F.Cu" "B.Cu") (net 11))
 (segment (start 102.536 95.33) (end 107.5 95.33) (width 0.5) (layer "B.Cu") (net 11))
 (segment (start 66.78 99.05) (end 66.73 99) (width 0.25) (layer "B.Cu") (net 11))
 (segment (start 89.221857 84.006143) (end 89.221857 77.523596) (width 0.5) (layer "B.Cu") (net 11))
 (segment (start 90.424 113.792) (end 89.779467 114.436533) (width 0.5) (layer "B.Cu") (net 11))
 (segment (start 74.8 99.05) (end 66.78 99.05) (width 0.5) (layer "B.Cu") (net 11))
 (segment (start 87.376 85.852) (end 89.221857 84.006143) (width 0.5) (layer "B.Cu") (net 11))
 (segment (start 89.779467 114.436533) (end 89.779467 121.250706) (width 0.5) (layer "B.Cu") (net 11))
 (segment (start 102.108 95.758) (end 102.536 95.33) (width 0.5) (layer "B.Cu") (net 11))
 (segment (start 138.486 119.634) (end 136.72 121.4) (width 0.5) (layer "B.Cu") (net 4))
 (segment (start 136.72 121.08) (end 136.72 121.4) (width 0.25) (layer "B.Cu") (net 4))
 (segment (start 151.169 119.634) (end 138.486 119.634) (width 0.5) (layer "B.Cu") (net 4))
 (segment (start 153.785 122.25) (end 151.169 119.634) (width 0.5) (layer "B.Cu") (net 4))
 (segment (start 154.94 116.84) (end 156.325 118.225) (width 0.5) (layer "B.Cu") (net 3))
 (segment (start 156.325 118.225) (end 156.325 122.25) (width 0.5) (layer "B.Cu") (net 3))
 (segment (start 134.18 121.4) (end 138.74 116.84) (width 0.5) (layer "B.Cu") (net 3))
 (segment (start 138.74 116.84) (end 154.94 116.84) (width 0.5) (layer "B.Cu") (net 3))
 (segment (start 79.68 93.9) (end 83.6 93.9) (width 0.5) (layer "F.Cu") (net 1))
 (segment (start 84.074 101.092) (end 83.6 100.618) (width 0.5) (layer "F.Cu") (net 1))
 (segment (start 83.6 100.618) (end 83.6 93.9) (width 0.5) (layer "F.Cu") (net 1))
 (segment (start 94.793872 93.9) (end 83.6 93.9) (width 0.5) (layer "F.Cu") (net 1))
 (segment (start 94.92 94.026128) (end 94.793872 93.9) (width 0.5) (layer "F.Cu") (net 1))
 (via (at 84.074 101.092) (size 1.5) (drill 1) (layers "F.Cu" "B.Cu") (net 1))
 (via (at 94.92 94.026128) (size 1.5) (drill 1) (layers "F.Cu" "B.Cu") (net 1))
 (via (at 79.68 93.9) (size 1.5) (drill 1) (layers "F.Cu" "B.Cu") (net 1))
 (segment (start 129.1 114.232) (end 129.1 121.4) (width 0.5) (layer "B.Cu") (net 1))
 (segment (start 79.66 93.92) (end 66.73 93.92) (width 0.5) (layer "B.Cu") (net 1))
 (segment (start 84.074 101.092) (end 84.776644 101.794644) (width 0.5) (layer "B.Cu") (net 1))
 (segment (start 100.9 83.316783) (end 94.22468 76.641463) (width 0.5) (layer "B.Cu") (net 1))
 (segment (start 176.585 107) (end 176.585 107.715) (width 0.5) (layer "B.Cu") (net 1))
 (segment (start 176.585 107.715) (end 171.524 112.776) (width 0.5) (layer "B.Cu") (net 1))
 (segment (start 100.9 90.4) (end 100.9 83.86) (width 0.5) (layer "B.Cu") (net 1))
 (segment (start 100.9 83.86) (end 100.9 83.316783) (width 0.5) (layer "B.Cu") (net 1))
 (segment (start 107.5 80.09) (end 104.67 80.09) (width 0.5) (layer "B.Cu") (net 1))
 (segment (start 104.67 80.09) (end 100.9 83.86) (width 0.5) (layer "B.Cu") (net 1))
 (segment (start 94.92 94.026128) (end 97.273872 94.026128) (width 0.5) (layer "B.Cu") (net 1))
 (segment (start 97.273872 94.026128) (end 100.9 90.4) (width 0.5) (layer "B.Cu") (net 1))
 (segment (start 130.556 112.776) (end 129.1 114.232) (width 0.5) (layer "B.Cu") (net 1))
 (segment (start 84.776644 101.794644) (end 84.776644 120.368573) (width 0.5) (layer "B.Cu") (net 1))
 (segment (start 171.524 112.776) (end 130.692 112.776) (width 0.5) (layer "B.Cu") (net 1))
 (segment (start 79.68 93.9) (end 79.66 93.92) (width 0.5) (layer "B.Cu") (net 1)))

